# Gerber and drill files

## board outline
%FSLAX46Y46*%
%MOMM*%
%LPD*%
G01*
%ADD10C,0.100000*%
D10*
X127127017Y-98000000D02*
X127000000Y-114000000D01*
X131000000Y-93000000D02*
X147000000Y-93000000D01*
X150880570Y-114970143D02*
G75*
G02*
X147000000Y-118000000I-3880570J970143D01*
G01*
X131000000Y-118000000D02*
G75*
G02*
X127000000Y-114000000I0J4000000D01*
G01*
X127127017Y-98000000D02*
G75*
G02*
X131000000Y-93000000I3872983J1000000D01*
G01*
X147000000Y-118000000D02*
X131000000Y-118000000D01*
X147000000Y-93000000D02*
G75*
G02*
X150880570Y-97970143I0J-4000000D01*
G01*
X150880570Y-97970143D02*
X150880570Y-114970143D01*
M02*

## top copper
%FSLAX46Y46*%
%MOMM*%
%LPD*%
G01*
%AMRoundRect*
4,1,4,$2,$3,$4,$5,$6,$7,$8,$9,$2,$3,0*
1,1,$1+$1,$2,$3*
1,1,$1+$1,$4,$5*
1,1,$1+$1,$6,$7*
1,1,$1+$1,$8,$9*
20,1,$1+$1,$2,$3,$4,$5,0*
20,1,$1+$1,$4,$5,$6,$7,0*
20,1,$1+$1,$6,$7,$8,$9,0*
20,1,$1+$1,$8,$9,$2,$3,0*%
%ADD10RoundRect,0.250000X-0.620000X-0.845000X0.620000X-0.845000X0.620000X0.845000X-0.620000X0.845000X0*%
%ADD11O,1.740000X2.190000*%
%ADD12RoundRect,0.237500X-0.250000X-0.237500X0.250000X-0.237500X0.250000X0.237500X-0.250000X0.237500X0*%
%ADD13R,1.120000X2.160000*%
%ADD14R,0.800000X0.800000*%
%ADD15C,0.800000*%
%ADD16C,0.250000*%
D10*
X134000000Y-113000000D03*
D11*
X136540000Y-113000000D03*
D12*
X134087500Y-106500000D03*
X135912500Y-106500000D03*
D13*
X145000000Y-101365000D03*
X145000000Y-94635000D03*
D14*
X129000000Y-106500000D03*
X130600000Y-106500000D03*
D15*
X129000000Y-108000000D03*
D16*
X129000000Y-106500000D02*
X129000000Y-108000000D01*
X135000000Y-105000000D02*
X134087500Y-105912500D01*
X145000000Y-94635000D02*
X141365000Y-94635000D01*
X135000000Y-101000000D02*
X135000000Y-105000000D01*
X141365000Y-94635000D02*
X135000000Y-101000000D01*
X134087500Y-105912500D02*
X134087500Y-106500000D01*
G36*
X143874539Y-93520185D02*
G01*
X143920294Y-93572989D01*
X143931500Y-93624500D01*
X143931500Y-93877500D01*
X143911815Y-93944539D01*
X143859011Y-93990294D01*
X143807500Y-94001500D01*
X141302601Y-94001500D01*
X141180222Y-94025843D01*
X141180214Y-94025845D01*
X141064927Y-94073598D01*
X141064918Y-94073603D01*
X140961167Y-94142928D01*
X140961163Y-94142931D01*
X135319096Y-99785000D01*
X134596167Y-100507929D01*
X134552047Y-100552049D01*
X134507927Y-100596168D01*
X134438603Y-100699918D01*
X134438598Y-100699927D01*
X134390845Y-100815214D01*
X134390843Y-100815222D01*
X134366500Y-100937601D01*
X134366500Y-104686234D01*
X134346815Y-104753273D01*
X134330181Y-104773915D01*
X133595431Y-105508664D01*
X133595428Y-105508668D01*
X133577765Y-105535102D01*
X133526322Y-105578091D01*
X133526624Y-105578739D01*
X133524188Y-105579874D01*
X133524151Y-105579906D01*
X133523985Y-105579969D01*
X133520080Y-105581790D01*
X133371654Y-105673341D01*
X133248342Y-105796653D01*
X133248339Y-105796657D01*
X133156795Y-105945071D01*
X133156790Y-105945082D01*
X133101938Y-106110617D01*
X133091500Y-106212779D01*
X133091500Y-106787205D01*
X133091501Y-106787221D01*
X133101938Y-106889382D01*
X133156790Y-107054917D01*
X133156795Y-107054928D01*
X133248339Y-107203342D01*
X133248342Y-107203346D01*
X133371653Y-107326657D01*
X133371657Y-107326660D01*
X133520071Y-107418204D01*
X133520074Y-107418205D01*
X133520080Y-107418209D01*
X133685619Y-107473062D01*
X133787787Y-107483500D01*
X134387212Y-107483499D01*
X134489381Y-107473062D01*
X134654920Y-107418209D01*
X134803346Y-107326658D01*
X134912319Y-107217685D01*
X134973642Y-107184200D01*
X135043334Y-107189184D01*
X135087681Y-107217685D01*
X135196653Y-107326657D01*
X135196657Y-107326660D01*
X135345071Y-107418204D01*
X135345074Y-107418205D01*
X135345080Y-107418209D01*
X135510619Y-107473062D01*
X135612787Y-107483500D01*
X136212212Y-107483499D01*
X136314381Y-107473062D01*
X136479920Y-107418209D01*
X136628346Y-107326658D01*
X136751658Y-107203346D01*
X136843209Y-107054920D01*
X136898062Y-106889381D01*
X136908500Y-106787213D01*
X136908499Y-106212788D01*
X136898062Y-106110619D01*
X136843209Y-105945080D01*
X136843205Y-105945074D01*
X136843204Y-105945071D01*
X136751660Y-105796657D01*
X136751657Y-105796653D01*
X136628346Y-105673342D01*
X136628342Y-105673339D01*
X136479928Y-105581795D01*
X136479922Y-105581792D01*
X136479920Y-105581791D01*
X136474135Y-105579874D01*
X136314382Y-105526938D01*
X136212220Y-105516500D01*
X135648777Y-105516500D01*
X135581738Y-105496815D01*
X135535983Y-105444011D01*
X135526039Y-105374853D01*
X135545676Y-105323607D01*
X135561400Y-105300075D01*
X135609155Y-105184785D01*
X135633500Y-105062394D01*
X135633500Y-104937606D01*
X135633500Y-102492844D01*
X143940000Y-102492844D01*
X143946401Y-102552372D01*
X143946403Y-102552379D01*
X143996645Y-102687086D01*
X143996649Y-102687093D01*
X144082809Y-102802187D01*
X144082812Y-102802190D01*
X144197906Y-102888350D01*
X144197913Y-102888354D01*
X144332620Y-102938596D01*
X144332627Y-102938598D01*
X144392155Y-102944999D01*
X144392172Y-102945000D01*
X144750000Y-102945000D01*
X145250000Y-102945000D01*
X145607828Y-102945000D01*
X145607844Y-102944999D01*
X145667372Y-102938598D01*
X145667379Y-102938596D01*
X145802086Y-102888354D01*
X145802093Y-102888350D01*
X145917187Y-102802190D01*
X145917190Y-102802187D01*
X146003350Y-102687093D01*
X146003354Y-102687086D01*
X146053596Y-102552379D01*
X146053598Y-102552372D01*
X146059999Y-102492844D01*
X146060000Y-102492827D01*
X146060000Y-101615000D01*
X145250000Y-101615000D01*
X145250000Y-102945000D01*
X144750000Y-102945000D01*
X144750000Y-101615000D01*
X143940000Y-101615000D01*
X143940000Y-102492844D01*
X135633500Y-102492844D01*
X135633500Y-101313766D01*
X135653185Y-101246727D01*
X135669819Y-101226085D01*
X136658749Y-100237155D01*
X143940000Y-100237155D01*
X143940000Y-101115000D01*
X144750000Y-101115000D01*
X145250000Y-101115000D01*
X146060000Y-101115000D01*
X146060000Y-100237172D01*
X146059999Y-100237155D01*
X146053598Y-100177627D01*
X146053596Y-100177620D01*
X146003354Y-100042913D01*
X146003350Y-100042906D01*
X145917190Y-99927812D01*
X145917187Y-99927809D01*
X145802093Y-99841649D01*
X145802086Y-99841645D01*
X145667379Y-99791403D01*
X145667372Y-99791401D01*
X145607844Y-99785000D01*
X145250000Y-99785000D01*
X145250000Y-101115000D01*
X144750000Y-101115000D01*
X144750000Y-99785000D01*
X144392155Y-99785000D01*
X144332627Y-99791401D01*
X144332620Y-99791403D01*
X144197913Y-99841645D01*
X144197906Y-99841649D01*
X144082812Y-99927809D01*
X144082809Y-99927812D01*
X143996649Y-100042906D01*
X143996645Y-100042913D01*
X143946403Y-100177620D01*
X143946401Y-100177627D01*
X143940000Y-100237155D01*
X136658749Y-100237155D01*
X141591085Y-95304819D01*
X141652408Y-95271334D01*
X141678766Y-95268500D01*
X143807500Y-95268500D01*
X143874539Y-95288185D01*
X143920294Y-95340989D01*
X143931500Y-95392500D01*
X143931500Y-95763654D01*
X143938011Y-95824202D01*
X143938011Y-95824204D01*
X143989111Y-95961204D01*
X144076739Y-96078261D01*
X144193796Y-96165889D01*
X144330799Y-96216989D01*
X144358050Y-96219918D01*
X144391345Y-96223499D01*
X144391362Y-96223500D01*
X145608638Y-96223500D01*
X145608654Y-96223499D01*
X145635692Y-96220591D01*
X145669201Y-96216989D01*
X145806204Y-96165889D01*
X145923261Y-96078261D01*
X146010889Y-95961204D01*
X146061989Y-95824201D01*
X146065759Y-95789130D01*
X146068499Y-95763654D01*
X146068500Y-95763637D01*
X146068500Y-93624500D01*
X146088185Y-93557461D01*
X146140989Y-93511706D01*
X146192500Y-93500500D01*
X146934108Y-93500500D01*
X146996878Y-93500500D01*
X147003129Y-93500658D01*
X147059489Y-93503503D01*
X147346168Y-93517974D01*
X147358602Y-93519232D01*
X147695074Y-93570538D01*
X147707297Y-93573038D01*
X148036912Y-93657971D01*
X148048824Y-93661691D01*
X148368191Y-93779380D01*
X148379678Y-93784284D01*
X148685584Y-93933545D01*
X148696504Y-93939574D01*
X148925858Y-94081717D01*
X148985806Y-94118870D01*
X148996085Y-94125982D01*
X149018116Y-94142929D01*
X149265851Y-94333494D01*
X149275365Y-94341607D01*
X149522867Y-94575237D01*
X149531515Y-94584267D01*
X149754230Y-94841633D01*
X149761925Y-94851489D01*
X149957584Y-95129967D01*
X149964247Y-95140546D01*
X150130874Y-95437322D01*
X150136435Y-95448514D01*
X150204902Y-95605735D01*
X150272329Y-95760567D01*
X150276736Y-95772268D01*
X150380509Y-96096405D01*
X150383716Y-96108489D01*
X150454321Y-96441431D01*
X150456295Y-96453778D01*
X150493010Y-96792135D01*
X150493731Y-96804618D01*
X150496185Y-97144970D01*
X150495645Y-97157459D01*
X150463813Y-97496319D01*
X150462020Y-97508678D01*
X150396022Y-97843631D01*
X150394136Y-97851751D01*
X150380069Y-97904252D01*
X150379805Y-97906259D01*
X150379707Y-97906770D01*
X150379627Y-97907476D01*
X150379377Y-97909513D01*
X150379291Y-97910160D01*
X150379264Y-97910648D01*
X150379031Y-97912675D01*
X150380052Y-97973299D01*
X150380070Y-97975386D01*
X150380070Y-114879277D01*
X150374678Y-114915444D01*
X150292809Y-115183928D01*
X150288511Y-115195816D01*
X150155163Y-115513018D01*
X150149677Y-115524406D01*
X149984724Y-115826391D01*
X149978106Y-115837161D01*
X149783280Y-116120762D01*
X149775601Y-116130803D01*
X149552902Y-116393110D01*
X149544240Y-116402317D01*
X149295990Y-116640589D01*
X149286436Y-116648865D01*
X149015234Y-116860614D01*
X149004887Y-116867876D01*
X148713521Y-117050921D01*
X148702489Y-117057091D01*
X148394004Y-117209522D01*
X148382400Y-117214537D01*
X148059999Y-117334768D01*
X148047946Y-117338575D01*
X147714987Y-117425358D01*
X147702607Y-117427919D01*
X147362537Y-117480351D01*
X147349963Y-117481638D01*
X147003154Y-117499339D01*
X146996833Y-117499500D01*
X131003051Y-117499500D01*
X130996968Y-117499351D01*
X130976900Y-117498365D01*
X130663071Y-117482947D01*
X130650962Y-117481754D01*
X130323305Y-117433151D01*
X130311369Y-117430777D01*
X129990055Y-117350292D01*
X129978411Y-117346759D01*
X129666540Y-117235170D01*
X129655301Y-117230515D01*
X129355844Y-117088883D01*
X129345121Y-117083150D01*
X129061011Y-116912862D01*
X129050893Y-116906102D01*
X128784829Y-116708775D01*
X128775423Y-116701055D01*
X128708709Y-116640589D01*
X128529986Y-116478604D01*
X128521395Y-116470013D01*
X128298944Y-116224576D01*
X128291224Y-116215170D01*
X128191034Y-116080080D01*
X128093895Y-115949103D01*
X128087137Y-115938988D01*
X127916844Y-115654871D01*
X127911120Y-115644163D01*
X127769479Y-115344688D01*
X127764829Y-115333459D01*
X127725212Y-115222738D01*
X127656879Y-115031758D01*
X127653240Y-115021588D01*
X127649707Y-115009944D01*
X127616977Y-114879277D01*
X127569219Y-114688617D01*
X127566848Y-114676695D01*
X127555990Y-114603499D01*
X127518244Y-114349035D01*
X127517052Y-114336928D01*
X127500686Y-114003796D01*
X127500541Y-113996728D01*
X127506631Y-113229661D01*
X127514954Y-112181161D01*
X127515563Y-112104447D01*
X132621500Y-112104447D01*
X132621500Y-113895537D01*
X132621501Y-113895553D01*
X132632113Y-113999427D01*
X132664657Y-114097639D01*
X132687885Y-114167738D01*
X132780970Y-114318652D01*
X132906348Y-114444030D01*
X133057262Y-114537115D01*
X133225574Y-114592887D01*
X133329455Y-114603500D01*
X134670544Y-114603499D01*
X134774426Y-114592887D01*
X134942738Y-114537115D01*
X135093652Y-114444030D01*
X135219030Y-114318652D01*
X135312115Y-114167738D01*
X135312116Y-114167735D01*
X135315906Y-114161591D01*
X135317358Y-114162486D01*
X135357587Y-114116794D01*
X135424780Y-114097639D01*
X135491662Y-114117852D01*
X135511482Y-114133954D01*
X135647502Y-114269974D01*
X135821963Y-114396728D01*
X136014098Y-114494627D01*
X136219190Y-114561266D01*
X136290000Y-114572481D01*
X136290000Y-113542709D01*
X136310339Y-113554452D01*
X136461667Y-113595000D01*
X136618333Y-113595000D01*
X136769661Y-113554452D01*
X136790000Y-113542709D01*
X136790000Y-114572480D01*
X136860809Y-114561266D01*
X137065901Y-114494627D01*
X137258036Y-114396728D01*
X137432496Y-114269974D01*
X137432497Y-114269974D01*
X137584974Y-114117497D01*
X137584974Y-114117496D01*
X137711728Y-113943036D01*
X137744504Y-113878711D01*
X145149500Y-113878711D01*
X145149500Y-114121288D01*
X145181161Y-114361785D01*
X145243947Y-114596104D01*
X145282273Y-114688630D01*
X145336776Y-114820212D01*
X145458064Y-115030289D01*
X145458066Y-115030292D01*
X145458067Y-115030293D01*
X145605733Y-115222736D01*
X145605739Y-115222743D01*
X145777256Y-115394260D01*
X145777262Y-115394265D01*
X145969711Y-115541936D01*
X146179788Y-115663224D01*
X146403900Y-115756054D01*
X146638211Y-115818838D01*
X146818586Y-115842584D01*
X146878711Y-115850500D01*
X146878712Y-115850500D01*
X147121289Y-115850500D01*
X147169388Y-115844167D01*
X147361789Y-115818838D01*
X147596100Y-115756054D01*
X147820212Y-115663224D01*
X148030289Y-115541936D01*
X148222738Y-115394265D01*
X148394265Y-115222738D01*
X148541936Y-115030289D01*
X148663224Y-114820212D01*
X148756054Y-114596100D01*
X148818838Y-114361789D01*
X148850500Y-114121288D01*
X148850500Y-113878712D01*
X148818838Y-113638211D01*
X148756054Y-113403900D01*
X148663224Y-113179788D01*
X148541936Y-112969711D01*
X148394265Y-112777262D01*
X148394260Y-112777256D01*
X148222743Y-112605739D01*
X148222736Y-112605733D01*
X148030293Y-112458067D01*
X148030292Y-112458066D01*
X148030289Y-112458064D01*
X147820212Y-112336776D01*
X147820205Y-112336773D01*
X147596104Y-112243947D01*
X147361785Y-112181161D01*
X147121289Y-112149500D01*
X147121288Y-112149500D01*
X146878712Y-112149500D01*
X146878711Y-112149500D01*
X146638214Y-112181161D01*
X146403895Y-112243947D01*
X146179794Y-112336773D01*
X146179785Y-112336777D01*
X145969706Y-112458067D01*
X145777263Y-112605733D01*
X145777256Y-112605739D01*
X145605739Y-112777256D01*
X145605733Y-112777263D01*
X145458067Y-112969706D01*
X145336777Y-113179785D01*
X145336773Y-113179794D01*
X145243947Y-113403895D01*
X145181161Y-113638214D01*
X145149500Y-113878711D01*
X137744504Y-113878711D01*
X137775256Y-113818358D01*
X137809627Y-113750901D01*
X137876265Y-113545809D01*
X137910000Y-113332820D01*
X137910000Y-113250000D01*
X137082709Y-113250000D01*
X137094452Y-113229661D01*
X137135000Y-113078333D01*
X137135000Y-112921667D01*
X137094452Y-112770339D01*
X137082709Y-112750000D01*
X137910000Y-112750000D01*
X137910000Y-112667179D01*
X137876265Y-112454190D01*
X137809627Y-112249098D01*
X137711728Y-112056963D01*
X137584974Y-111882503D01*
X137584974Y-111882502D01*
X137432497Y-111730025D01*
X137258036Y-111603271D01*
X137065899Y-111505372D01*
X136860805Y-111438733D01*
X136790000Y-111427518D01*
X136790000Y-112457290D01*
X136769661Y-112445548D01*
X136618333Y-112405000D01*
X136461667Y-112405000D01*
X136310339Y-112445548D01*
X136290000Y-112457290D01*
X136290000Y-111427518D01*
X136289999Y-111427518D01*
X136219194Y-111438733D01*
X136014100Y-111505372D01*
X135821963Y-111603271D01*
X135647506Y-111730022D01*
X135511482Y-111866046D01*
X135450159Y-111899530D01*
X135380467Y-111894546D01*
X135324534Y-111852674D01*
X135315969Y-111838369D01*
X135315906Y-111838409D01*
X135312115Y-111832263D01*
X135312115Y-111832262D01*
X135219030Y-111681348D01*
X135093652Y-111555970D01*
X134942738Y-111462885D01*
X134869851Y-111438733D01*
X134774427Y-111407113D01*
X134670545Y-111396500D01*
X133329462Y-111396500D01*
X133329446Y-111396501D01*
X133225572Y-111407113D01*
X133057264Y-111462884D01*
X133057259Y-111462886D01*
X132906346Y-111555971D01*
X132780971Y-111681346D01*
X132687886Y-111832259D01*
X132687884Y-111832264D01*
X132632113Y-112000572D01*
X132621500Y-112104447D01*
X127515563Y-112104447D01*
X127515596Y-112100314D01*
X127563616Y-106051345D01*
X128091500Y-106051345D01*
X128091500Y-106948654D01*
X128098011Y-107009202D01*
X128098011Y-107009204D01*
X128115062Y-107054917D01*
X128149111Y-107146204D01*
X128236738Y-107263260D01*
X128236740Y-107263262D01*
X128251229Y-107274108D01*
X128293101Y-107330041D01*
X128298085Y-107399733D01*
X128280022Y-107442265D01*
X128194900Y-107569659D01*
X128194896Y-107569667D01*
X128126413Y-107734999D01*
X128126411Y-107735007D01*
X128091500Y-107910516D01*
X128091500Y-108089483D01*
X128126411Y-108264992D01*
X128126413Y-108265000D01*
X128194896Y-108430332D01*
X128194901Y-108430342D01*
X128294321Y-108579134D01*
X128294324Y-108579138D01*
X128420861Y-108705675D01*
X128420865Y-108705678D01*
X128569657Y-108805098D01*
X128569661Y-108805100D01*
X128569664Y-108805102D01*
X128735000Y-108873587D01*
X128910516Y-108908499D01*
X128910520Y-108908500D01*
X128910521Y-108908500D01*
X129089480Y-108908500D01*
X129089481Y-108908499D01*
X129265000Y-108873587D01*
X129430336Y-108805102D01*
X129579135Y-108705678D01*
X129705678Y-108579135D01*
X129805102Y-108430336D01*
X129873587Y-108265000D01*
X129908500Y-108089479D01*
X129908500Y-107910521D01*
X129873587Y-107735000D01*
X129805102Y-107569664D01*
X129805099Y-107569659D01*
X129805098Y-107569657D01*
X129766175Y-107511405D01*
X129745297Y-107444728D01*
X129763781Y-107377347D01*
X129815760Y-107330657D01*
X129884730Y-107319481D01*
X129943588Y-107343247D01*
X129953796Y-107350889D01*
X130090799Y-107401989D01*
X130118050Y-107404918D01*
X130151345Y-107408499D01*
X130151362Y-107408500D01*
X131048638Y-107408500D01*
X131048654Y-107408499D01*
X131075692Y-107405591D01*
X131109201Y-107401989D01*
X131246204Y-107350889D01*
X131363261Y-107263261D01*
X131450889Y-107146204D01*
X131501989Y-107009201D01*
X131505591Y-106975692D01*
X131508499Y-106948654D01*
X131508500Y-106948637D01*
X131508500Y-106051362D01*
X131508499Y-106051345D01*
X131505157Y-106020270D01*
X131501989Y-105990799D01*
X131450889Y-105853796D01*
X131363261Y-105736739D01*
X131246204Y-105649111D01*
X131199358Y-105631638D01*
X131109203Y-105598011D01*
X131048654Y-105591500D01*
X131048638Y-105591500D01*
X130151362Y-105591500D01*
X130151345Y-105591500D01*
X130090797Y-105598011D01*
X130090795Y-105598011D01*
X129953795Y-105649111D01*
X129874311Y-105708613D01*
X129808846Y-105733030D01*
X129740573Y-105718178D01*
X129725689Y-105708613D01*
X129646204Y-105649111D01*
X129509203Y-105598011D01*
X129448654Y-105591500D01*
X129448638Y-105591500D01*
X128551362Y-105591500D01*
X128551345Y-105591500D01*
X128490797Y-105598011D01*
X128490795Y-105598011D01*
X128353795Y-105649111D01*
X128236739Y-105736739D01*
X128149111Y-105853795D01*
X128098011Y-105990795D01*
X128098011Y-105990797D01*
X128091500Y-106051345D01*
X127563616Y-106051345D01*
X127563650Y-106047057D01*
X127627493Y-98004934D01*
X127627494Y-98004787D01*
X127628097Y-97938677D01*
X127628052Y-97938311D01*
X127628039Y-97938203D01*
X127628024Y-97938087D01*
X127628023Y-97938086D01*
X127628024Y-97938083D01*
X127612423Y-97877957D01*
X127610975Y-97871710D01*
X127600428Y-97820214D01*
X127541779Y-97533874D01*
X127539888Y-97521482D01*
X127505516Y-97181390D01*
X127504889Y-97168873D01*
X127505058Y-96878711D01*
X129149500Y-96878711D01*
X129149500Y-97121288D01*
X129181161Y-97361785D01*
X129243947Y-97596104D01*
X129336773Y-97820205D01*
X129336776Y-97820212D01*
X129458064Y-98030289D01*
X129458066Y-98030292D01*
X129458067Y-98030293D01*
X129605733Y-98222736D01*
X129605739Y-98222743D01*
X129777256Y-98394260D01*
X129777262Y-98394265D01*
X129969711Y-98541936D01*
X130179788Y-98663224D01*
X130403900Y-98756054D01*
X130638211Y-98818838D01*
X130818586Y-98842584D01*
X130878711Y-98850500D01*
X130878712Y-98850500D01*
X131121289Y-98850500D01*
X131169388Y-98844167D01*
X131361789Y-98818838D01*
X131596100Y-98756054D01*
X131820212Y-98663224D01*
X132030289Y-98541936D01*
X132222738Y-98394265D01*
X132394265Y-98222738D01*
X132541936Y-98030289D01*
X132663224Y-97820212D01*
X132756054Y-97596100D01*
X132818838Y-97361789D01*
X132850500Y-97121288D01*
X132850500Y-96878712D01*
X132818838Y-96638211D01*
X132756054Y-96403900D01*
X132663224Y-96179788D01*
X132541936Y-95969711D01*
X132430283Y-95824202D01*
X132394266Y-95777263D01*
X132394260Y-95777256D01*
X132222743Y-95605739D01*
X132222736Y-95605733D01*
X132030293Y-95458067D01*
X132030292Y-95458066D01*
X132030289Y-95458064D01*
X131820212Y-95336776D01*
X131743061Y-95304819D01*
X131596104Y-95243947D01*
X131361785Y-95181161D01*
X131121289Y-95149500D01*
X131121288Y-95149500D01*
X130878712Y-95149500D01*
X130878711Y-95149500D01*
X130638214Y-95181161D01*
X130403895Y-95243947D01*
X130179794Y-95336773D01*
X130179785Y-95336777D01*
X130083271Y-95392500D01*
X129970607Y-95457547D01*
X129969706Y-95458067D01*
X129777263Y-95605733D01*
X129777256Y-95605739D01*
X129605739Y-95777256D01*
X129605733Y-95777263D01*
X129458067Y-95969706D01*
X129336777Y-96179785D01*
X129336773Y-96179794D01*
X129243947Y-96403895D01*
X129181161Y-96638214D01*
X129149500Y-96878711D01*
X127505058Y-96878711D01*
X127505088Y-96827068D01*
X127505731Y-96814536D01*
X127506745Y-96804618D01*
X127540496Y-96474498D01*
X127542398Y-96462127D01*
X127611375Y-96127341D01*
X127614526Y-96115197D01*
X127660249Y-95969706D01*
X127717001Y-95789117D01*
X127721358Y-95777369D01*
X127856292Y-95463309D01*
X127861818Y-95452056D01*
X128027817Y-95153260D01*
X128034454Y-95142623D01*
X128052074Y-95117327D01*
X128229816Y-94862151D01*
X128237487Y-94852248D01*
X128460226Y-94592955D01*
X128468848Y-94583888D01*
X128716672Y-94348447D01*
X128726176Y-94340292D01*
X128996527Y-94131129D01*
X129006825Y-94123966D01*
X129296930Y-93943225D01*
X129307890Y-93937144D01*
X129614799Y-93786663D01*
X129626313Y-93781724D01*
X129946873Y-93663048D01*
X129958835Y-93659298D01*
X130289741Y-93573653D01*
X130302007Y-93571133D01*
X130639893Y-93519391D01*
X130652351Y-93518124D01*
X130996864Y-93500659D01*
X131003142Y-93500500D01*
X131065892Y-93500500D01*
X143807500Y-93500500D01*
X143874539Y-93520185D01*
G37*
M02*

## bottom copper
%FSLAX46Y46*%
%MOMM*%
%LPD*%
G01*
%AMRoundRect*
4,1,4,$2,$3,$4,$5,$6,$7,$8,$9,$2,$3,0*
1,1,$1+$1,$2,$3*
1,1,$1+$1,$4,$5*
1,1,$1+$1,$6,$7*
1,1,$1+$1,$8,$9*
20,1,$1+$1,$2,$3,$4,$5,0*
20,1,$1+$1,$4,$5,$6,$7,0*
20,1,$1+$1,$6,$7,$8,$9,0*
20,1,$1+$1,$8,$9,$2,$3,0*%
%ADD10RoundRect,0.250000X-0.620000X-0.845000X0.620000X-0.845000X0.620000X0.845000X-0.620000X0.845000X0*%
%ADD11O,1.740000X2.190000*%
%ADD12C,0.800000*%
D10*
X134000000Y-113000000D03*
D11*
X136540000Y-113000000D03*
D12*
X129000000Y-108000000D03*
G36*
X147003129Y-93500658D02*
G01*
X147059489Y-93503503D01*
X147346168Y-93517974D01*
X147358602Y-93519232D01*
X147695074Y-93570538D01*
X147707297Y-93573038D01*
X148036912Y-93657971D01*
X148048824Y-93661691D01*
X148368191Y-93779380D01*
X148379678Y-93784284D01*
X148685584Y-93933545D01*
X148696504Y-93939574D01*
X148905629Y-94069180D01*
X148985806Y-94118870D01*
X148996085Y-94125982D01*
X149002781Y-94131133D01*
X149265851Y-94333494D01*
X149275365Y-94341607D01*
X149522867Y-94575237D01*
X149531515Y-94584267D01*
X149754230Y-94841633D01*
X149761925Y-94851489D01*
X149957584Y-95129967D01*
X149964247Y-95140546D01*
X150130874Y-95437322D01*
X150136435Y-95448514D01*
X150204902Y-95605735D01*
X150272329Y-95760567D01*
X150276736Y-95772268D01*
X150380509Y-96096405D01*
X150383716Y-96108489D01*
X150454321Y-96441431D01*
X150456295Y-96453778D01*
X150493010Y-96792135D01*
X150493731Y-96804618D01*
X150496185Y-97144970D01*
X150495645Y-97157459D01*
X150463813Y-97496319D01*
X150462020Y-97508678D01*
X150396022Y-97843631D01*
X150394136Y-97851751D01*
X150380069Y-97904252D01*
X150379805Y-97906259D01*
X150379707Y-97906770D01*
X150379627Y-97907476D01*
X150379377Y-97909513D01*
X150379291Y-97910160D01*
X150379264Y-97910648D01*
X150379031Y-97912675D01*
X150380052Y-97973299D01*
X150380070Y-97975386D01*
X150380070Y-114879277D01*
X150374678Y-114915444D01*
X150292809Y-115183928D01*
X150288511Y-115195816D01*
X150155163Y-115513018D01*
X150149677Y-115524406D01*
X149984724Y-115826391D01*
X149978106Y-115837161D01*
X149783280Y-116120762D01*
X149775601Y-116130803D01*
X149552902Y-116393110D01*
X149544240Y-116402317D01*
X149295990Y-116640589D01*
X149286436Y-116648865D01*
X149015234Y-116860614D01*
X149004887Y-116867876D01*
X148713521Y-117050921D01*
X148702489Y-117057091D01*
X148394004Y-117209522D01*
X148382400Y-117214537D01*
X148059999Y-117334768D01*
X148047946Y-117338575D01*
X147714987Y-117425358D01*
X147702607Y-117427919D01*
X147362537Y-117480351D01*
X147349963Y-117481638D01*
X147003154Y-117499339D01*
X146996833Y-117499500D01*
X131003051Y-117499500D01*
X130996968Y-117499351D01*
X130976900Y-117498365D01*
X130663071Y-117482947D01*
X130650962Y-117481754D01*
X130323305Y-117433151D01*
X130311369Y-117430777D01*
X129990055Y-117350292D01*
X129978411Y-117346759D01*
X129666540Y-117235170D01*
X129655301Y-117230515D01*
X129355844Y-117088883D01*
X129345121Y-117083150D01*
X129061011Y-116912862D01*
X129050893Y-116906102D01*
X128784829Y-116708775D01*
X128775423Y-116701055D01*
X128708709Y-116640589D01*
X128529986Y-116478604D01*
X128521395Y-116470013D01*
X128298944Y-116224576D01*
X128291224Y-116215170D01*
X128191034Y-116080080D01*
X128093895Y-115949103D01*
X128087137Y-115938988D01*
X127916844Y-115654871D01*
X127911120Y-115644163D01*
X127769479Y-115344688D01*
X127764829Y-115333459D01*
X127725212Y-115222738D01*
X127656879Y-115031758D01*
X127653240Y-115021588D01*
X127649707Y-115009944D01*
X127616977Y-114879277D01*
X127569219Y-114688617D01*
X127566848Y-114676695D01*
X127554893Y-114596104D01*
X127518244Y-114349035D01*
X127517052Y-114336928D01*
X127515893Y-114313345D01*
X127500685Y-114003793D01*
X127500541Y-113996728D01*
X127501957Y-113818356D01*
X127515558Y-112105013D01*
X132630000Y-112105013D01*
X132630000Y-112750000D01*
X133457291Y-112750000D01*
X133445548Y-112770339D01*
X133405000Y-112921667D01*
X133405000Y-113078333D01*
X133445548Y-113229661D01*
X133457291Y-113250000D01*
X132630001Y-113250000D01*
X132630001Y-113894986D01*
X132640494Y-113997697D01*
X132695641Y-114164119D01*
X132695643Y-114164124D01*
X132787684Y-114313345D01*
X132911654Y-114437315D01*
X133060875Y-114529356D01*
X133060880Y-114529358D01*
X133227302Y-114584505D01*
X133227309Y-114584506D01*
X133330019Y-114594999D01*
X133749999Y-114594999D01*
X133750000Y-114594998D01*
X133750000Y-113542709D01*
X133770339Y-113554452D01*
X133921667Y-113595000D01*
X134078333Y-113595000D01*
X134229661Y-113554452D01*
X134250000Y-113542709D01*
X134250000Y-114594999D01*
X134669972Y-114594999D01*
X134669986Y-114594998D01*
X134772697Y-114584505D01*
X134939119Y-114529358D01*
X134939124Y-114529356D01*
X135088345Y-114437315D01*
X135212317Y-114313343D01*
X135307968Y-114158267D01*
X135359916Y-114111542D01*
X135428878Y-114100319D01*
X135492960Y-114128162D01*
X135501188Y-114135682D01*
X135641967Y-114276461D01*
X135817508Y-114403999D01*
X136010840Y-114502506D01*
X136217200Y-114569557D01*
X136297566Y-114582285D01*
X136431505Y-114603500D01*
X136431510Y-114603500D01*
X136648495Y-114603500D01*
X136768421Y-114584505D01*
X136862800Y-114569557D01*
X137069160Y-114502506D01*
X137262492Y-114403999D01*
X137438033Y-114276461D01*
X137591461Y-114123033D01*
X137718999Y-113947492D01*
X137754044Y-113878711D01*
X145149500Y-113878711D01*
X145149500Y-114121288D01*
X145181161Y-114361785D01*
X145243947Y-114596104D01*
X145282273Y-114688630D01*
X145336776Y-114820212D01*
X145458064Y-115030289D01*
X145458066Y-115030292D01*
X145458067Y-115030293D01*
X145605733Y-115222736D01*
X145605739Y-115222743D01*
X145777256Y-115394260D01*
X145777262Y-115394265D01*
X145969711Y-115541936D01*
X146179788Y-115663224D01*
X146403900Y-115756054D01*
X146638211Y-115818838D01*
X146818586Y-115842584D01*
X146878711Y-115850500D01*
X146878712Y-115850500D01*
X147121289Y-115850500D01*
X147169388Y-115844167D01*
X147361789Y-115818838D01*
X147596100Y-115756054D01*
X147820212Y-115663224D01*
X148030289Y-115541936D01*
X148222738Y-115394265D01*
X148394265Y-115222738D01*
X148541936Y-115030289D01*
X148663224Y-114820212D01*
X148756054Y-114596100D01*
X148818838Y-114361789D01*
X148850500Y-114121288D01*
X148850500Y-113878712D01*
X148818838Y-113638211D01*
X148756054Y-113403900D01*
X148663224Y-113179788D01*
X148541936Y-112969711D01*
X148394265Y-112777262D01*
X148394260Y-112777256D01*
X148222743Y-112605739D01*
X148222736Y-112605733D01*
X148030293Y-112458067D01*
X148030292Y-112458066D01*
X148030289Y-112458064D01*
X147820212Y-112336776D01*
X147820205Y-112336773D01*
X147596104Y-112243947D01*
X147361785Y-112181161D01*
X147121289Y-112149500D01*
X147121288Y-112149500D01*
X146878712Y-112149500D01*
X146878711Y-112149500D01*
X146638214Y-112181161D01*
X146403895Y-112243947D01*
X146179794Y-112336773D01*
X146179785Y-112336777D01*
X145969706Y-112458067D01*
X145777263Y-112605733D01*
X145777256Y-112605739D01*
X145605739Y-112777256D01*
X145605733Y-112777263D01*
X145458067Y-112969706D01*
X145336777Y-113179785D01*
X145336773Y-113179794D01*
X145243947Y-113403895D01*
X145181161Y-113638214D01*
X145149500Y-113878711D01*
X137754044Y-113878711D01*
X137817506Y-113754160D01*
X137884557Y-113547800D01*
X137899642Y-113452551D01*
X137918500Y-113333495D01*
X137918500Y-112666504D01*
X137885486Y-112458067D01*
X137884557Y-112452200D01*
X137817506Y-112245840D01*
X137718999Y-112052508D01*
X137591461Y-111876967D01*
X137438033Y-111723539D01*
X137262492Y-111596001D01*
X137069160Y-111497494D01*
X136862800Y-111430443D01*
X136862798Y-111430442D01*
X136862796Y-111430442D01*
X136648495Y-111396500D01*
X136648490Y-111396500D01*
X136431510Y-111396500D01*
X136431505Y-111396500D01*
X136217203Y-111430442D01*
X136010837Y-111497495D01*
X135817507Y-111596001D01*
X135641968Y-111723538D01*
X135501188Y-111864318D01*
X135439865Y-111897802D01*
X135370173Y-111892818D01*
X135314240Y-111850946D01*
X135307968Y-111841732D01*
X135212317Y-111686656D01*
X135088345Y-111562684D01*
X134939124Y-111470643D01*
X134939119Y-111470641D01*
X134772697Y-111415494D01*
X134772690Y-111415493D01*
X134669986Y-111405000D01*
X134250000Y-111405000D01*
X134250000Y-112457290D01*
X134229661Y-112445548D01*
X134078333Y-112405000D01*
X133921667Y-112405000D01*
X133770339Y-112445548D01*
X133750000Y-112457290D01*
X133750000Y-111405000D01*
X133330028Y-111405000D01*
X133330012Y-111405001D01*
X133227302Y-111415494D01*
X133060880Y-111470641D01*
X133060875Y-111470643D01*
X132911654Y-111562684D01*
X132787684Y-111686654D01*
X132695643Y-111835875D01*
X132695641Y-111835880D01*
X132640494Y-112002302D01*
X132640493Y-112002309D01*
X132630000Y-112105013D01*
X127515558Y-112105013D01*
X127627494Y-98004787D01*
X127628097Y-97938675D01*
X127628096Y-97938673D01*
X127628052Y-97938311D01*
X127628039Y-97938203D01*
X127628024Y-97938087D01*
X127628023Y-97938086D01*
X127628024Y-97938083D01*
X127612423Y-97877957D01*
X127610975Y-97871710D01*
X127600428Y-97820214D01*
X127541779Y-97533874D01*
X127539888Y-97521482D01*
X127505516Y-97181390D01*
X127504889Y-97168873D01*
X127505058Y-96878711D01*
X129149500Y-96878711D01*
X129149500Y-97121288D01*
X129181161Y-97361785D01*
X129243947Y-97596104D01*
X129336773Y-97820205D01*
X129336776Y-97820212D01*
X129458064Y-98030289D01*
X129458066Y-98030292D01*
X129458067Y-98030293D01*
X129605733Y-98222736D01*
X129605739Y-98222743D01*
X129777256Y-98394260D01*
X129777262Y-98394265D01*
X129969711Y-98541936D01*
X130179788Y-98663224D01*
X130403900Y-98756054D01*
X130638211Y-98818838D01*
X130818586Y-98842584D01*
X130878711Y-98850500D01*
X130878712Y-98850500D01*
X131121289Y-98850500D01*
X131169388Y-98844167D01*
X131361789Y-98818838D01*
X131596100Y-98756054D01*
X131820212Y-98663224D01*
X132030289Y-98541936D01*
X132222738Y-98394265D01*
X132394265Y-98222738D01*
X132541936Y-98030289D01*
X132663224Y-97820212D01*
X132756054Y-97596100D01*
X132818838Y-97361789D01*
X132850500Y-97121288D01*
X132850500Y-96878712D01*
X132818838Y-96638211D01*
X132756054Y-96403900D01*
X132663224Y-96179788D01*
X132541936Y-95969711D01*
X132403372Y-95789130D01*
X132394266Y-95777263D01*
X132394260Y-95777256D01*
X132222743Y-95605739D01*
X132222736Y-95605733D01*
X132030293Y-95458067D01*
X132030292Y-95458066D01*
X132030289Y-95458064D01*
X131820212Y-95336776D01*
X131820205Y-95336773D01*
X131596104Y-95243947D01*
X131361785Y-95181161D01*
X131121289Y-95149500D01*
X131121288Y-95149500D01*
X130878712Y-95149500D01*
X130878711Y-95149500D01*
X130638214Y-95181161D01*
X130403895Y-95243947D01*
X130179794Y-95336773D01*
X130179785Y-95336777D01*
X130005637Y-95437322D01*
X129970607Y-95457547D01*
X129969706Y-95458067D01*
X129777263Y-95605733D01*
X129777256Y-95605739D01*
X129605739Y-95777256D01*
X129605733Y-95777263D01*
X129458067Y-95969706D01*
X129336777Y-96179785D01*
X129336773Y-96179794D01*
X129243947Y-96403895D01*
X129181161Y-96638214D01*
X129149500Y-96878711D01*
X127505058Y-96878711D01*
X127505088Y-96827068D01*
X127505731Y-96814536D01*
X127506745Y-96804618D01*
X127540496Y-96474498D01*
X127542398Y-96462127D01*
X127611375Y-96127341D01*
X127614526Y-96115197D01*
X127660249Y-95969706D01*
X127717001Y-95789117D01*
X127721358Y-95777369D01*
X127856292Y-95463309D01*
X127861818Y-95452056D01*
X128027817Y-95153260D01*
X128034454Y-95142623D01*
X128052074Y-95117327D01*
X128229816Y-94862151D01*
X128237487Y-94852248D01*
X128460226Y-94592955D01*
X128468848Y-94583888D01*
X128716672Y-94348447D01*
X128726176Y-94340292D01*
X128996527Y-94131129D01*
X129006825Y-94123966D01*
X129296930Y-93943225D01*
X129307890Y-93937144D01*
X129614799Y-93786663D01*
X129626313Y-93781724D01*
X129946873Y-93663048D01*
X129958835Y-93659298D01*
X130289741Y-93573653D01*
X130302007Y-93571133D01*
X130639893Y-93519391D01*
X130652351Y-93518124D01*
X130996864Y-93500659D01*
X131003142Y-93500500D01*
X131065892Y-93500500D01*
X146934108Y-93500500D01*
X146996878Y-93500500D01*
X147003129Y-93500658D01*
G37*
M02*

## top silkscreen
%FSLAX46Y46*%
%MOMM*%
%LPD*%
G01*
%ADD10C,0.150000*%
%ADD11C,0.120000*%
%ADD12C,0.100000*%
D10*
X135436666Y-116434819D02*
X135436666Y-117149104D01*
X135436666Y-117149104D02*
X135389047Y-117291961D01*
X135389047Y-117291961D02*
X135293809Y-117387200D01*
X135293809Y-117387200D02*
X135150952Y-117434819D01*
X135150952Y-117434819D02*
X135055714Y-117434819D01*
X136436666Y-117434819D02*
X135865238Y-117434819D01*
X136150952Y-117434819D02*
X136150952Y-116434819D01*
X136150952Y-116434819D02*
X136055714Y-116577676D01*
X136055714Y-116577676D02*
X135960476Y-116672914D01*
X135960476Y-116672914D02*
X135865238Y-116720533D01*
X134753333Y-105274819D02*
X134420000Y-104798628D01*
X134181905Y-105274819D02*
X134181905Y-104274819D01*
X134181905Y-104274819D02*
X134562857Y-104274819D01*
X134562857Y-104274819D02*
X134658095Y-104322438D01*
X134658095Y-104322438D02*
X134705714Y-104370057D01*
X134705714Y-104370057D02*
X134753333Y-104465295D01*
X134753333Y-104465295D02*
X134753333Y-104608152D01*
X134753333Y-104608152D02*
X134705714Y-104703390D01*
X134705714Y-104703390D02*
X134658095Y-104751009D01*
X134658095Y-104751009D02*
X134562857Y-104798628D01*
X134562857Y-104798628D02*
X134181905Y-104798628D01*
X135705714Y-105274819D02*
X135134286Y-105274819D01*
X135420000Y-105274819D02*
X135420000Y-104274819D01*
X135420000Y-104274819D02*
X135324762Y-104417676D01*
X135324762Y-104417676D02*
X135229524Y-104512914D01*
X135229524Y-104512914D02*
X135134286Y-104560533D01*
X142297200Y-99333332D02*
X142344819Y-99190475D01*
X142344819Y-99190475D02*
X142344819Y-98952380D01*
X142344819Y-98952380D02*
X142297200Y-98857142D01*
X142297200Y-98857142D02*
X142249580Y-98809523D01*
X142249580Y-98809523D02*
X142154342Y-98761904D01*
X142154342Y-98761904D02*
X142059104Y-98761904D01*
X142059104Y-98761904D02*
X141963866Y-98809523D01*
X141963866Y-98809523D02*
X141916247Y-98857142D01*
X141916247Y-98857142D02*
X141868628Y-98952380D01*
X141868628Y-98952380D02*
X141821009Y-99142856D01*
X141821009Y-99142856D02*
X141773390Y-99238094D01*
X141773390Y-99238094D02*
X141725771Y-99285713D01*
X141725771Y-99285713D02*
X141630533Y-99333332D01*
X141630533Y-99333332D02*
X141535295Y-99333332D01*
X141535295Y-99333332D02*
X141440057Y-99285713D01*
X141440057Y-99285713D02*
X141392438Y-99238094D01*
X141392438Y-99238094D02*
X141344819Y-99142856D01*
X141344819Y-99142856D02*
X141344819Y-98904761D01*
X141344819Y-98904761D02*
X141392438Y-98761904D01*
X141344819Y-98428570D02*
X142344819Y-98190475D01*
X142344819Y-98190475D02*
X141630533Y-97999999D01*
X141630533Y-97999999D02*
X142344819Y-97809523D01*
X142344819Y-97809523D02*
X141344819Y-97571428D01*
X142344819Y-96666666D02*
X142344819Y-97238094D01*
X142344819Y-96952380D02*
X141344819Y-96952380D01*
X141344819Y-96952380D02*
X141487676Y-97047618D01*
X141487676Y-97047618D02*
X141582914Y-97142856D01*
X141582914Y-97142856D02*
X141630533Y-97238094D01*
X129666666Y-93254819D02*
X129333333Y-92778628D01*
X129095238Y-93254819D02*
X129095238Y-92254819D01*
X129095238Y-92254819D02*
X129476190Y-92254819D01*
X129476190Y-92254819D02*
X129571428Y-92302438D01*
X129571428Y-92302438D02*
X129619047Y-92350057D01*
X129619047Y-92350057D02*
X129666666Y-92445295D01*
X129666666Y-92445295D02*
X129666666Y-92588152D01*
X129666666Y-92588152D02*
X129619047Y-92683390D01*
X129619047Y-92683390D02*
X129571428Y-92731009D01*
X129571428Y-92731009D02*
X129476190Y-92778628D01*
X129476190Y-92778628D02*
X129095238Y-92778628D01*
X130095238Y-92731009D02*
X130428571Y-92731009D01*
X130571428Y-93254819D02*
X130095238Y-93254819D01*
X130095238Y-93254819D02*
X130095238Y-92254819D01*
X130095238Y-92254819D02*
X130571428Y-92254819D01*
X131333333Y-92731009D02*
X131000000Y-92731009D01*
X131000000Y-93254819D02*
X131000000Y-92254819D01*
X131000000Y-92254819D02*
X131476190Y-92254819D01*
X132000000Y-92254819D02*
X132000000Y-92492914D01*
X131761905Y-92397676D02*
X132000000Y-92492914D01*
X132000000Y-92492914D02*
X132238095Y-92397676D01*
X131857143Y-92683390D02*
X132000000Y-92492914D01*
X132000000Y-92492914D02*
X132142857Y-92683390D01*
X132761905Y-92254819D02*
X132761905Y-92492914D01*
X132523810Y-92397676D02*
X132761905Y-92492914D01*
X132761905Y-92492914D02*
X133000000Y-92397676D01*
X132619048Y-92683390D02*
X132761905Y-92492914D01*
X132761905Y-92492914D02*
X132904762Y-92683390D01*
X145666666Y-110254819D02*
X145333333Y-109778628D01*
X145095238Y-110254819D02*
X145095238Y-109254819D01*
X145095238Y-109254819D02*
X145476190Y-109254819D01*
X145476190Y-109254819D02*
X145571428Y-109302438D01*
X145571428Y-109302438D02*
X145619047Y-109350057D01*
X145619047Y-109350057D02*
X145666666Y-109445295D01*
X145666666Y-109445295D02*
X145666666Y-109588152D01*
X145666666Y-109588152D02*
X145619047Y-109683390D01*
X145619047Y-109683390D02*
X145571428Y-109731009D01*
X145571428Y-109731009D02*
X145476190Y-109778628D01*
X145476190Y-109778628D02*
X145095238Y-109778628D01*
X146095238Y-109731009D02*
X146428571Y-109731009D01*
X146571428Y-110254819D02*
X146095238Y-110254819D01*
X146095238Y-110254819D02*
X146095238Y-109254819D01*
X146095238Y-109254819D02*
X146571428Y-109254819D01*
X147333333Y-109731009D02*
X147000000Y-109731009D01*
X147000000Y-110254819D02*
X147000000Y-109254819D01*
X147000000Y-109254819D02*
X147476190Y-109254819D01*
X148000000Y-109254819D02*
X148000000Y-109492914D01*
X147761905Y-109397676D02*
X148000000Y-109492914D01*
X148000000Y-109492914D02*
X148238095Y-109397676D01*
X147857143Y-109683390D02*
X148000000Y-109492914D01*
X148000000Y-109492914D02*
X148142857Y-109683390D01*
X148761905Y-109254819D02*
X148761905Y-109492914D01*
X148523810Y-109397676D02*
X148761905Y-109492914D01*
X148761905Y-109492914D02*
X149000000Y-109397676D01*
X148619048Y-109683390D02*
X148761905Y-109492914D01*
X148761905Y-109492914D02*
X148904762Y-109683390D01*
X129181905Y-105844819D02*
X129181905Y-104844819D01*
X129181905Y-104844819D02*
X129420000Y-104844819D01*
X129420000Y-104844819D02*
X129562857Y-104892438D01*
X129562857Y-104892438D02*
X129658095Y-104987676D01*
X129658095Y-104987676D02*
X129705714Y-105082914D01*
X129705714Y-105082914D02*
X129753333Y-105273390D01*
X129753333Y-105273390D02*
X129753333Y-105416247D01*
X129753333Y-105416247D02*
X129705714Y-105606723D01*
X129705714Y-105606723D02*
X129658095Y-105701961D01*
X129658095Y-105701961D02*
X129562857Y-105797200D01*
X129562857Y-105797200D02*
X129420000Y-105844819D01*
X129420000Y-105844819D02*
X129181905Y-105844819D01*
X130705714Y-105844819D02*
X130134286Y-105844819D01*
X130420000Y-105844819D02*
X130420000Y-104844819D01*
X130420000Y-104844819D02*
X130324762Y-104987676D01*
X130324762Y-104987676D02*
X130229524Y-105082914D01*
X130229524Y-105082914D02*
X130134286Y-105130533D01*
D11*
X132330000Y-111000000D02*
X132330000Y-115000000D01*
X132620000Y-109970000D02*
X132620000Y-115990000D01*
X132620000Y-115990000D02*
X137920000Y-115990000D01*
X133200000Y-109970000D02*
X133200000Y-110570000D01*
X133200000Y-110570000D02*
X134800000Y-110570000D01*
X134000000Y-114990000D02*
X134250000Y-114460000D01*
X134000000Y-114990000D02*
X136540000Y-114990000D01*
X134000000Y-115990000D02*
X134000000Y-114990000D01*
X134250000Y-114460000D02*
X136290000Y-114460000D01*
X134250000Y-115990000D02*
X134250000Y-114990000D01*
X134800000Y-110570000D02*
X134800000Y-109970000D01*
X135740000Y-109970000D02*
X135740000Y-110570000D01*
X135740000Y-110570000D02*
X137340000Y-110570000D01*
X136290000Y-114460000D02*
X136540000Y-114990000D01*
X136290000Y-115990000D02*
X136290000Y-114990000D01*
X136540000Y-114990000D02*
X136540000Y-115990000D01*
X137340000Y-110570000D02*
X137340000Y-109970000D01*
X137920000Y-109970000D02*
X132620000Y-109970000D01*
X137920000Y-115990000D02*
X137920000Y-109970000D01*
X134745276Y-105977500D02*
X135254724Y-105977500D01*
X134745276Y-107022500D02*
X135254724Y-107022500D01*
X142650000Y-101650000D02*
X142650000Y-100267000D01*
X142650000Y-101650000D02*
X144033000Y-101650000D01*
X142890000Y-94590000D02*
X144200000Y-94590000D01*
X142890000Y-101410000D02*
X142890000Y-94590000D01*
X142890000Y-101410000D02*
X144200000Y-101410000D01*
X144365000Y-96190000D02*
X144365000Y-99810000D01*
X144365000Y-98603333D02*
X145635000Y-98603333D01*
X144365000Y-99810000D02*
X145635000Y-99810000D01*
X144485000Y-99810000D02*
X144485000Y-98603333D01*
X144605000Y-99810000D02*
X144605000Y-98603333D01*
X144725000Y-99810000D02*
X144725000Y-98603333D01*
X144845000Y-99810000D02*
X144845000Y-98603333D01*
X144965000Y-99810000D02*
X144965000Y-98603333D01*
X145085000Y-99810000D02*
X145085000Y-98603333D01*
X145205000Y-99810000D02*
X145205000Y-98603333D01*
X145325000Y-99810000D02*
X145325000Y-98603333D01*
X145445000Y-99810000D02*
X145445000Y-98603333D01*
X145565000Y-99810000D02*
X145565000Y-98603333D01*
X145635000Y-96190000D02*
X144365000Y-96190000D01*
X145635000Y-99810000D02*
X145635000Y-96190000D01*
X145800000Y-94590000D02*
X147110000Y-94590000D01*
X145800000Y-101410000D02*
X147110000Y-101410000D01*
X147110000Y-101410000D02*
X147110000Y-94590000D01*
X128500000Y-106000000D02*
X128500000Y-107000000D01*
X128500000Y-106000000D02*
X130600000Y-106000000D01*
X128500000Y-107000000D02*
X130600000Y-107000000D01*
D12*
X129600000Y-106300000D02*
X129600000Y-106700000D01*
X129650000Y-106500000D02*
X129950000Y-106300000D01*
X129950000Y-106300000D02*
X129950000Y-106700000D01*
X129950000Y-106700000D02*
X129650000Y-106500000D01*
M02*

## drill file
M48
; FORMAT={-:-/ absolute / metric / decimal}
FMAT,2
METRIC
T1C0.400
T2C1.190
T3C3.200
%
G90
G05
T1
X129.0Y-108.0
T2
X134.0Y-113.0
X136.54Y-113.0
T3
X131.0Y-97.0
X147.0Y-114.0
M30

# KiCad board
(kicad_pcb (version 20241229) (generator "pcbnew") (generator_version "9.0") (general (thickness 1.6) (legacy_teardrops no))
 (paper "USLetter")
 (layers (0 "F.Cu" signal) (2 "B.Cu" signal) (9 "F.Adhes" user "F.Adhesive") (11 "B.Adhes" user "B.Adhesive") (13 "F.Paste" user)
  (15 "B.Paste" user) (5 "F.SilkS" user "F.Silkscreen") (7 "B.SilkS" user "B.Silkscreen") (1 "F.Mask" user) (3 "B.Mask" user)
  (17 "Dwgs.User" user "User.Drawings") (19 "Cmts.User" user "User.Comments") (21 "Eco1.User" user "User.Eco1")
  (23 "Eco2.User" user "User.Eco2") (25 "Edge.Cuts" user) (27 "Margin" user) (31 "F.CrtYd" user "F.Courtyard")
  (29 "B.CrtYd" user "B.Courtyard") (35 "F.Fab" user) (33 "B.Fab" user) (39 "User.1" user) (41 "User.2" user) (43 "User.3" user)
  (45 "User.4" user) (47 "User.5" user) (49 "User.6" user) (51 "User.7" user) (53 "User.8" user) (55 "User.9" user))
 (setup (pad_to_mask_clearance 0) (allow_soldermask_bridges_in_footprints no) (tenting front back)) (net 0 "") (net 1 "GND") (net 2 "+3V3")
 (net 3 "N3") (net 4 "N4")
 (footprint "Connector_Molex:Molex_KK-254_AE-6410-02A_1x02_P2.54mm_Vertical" (layer "F.Cu") (at 134 113)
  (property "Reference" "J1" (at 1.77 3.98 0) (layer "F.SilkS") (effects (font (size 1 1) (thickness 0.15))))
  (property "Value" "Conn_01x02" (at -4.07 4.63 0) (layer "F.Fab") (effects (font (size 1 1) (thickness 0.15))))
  (fp_line (start -1.67 -2) (end -1.67 2) (stroke (width 0.12) (type solid)) (layer "F.SilkS"))
  (fp_line (start -1.38 -3.03) (end -1.38 2.99) (stroke (width 0.12) (type solid)) (layer "F.SilkS"))
  (fp_line (start -1.38 2.99) (end 3.92 2.99) (stroke (width 0.12) (type solid)) (layer "F.SilkS"))
  (fp_line (start -0.8 -3.03) (end -0.8 -2.43) (stroke (width 0.12) (type solid)) (layer "F.SilkS"))
  (fp_line (start -0.8 -2.43) (end 0.8 -2.43) (stroke (width 0.12) (type solid)) (layer "F.SilkS"))
  (fp_line (start 0 1.99) (end 0.25 1.46) (stroke (width 0.12) (type solid)) (layer "F.SilkS"))
  (fp_line (start 0 1.99) (end 2.54 1.99) (stroke (width 0.12) (type solid)) (layer "F.SilkS"))
  (fp_line (start 0 2.99) (end 0 1.99) (stroke (width 0.12) (type solid)) (layer "F.SilkS"))
  (fp_line (start 0.25 1.46) (end 2.29 1.46) (stroke (width 0.12) (type solid)) (layer "F.SilkS"))
  (fp_line (start 0.25 2.99) (end 0.25 1.99) (stroke (width 0.12) (type solid)) (layer "F.SilkS"))
  (fp_line (start 0.8 -2.43) (end 0.8 -3.03) (stroke (width 0.12) (type solid)) (layer "F.SilkS"))
  (fp_line (start 1.74 -3.03) (end 1.74 -2.43) (stroke (width 0.12) (type solid)) (layer "F.SilkS"))
  (fp_line (start 1.74 -2.43) (end 3.34 -2.43) (stroke (width 0.12) (type solid)) (layer "F.SilkS"))
  (fp_line (start 2.29 1.46) (end 2.54 1.99) (stroke (width 0.12) (type solid)) (layer "F.SilkS"))
  (fp_line (start 2.29 2.99) (end 2.29 1.99) (stroke (width 0.12) (type solid)) (layer "F.SilkS"))
  (fp_line (start 2.54 1.99) (end 2.54 2.99) (stroke (width 0.12) (type solid)) (layer "F.SilkS"))
  (fp_line (start 3.34 -2.43) (end 3.34 -3.03) (stroke (width 0.12) (type solid)) (layer "F.SilkS"))
  (fp_line (start 3.92 -3.03) (end -1.38 -3.03) (stroke (width 0.12) (type solid)) (layer "F.SilkS"))
  (fp_line (start 3.92 2.99) (end 3.92 -3.03) (stroke (width 0.12) (type solid)) (layer "F.SilkS"))
  (pad "1" thru_hole roundrect (at 0 0) (size 1.74 2.19) (drill 1.19) (layers "*.Cu" "*.Mask") (remove_unused_layers no)
   (roundrect_rratio 0.143678) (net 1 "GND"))
  (pad "2" thru_hole oval (at 2.54 0) (size 1.74 2.19) (drill 1.19) (layers "*.Cu" "*.Mask") (remove_unused_layers no) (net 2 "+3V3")))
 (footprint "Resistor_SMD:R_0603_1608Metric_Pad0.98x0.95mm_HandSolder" (layer "F.Cu") (at 135 106.5)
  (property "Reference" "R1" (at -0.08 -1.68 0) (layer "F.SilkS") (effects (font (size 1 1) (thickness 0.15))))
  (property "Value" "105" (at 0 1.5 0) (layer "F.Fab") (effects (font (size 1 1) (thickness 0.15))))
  (fp_line (start -0.254724 -0.5225) (end 0.254724 -0.5225) (stroke (width 0.12) (type solid)) (layer "F.SilkS"))
  (fp_line (start -0.254724 0.5225) (end 0.254724 0.5225) (stroke (width 0.12) (type solid)) (layer "F.SilkS"))
  (pad "1" smd roundrect (at -0.9125 0) (size 0.975 0.95) (layers "F.Cu" "F.Mask" "F.Paste") (roundrect_rratio 0.25) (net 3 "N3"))
  (pad "2" smd roundrect (at 0.9125 0) (size 0.975 0.95) (layers "F.Cu" "F.Mask" "F.Paste") (roundrect_rratio 0.25) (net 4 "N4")))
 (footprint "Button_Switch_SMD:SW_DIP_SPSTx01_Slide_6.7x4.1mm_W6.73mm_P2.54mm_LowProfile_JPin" (layer "F.Cu") (at 145 98 90)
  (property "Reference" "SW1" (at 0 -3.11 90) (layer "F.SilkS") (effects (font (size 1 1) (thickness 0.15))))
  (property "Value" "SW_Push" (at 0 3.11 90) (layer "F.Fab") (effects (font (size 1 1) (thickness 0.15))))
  (fp_line (start -3.65 -2.35) (end -2.267 -2.35) (stroke (width 0.12) (type solid)) (layer "F.SilkS"))
  (fp_line (start -3.65 -2.35) (end -3.65 -0.967) (stroke (width 0.12) (type solid)) (layer "F.SilkS"))
  (fp_line (start 3.41 -2.11) (end 3.41 -0.8) (stroke (width 0.12) (type solid)) (layer "F.SilkS"))
  (fp_line (start -3.41 -2.11) (end 3.41 -2.11) (stroke (width 0.12) (type solid)) (layer "F.SilkS"))
  (fp_line (start -3.41 -2.11) (end -3.41 -0.8) (stroke (width 0.12) (type solid)) (layer "F.SilkS"))
  (fp_line (start 1.81 -0.635) (end -1.81 -0.635) (stroke (width 0.12) (type solid)) (layer "F.SilkS"))
  (fp_line (start -0.603333 -0.635) (end -0.603333 0.635) (stroke (width 0.12) (type solid)) (layer "F.SilkS"))
  (fp_line (start -1.81 -0.635) (end -1.81 0.635) (stroke (width 0.12) (type solid)) (layer "F.SilkS"))
  (fp_line (start -1.81 -0.515) (end -0.603333 -0.515) (stroke (width 0.12) (type solid)) (layer "F.SilkS"))
  (fp_line (start -1.81 -0.395) (end -0.603333 -0.395) (stroke (width 0.12) (type solid)) (layer "F.SilkS"))
  (fp_line (start -1.81 -0.275) (end -0.603333 -0.275) (stroke (width 0.12) (type solid)) (layer "F.SilkS"))
  (fp_line (start -1.81 -0.155) (end -0.603333 -0.155) (stroke (width 0.12) (type solid)) (layer "F.SilkS"))
  (fp_line (start -1.81 -0.035) (end -0.603333 -0.035) (stroke (width 0.12) (type solid)) (layer "F.SilkS"))
  (fp_line (start -1.81 0.085) (end -0.603333 0.085) (stroke (width 0.12) (type solid)) (layer "F.SilkS"))
  (fp_line (start -1.81 0.205) (end -0.603333 0.205) (stroke (width 0.12) (type solid)) (layer "F.SilkS"))
  (fp_line (start -1.81 0.325) (end -0.603333 0.325) (stroke (width 0.12) (type solid)) (layer "F.SilkS"))
  (fp_line (start -1.81 0.445) (end -0.603333 0.445) (stroke (width 0.12) (type solid)) (layer "F.SilkS"))
  (fp_line (start -1.81 0.565) (end -0.603333 0.565) (stroke (width 0.12) (type solid)) (layer "F.SilkS"))
  (fp_line (start 1.81 0.635) (end 1.81 -0.635) (stroke (width 0.12) (type solid)) (layer "F.SilkS"))
  (fp_line (start -1.81 0.635) (end 1.81 0.635) (stroke (width 0.12) (type solid)) (layer "F.SilkS"))
  (fp_line (start 3.41 0.8) (end 3.41 2.11) (stroke (width 0.12) (type solid)) (layer "F.SilkS"))
  (fp_line (start -3.41 0.8) (end -3.41 2.11) (stroke (width 0.12) (type solid)) (layer "F.SilkS"))
  (fp_line (start -3.41 2.11) (end 3.41 2.11) (stroke (width 0.12) (type solid)) (layer "F.SilkS"))
  (pad "1" smd rect (at -3.365 0 90) (size 2.16 1.12) (layers "F.Cu" "F.Mask" "F.Paste") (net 2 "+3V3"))
  (pad "2" smd rect (at 3.365 0 90) (size 2.16 1.12) (layers "F.Cu" "F.Mask" "F.Paste") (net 3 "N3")))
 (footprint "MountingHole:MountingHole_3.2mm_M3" (layer "F.Cu") (at 131 97)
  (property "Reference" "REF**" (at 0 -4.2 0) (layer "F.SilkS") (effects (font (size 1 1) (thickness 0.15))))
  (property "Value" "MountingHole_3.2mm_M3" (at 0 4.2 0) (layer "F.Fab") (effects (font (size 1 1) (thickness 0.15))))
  (pad "" np_thru_hole circle (at 0 0) (size 3.2 3.2) (drill 3.2) (layers "*.Cu" "*.Mask")))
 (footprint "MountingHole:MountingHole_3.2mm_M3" (layer "F.Cu") (at 147 114)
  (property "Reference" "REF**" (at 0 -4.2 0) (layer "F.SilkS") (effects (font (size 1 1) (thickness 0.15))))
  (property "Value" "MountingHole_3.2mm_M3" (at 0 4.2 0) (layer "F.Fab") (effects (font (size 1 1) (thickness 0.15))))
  (pad "" np_thru_hole circle (at 0 0) (size 3.2 3.2) (drill 3.2) (layers "*.Cu" "*.Mask")))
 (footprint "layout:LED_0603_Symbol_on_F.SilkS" (layer "F.Cu") (at 129.8 106.5)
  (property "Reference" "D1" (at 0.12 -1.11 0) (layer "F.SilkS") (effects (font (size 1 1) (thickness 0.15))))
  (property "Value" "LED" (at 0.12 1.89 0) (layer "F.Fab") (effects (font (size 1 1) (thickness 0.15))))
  (fp_line (start -1.3 -0.5) (end -1.3 0.5) (stroke (width 0.12) (type solid)) (layer "F.SilkS"))
  (fp_line (start -1.3 -0.5) (end 0.8 -0.5) (stroke (width 0.12) (type solid)) (layer "F.SilkS"))
  (fp_line (start -1.3 0.5) (end 0.8 0.5) (stroke (width 0.12) (type solid)) (layer "F.SilkS"))
  (fp_line (start -0.2 -0.2) (end -0.2 0.2) (stroke (width 0.1) (type solid)) (layer "F.SilkS"))
  (fp_line (start -0.15 0) (end 0.15 -0.2) (stroke (width 0.1) (type solid)) (layer "F.SilkS"))
  (fp_line (start 0.15 -0.2) (end 0.15 0.2) (stroke (width 0.1) (type solid)) (layer "F.SilkS"))
  (fp_line (start 0.15 0.2) (end -0.15 0) (stroke (width 0.1) (type solid)) (layer "F.SilkS"))
  (pad "1" smd rect (at -0.8 0 180) (size 0.8 0.8) (layers "F.Cu" "F.Mask" "F.Paste") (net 1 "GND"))
  (pad "2" smd rect (at 0.8 0 180) (size 0.8 0.8) (layers "F.Cu" "F.Mask" "F.Paste") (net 4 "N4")))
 (gr_line (start 127.127017 98) (end 127 114) (stroke (width 0.1) (type default)) (layer "Edge.Cuts"))
 (gr_line (start 131 93) (end 147 93) (stroke (width 0.1) (type default)) (layer "Edge.Cuts"))
 (gr_arc (start 150.88057 114.970143) (mid 149.461649 117.152822) (end 147 118) (stroke (width 0.1) (type default)) (layer "Edge.Cuts"))
 (gr_arc (start 131 118) (mid 128.171573 116.828427) (end 127 114) (stroke (width 0.1) (type default)) (layer "Edge.Cuts"))
 (gr_arc (start 127.127017 98) (mid 127.837723 94.55051) (end 131 93) (stroke (width 0.1) (type default)) (layer "Edge.Cuts"))
 (gr_line (start 147 118) (end 131 118) (stroke (width 0.1) (type default)) (layer "Edge.Cuts"))
 (gr_arc (start 147 93) (mid 150.152822 94.538351) (end 150.88057 97.970143) (stroke (width 0.1) (type default)) (layer "Edge.Cuts"))
 (gr_line (start 150.88057 97.970143) (end 150.88057 114.970143) (stroke (width 0.1) (type default)) (layer "Edge.Cuts"))
 (segment (start 129 106.5) (end 129 108) (width 0.25) (layer "F.Cu") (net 1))
 (via (at 129 108) (size 0.8) (drill 0.4) (layers "F.Cu" "B.Cu") (free yes) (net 1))
 (segment (start 135 105) (end 134.0875 105.9125) (width 0.25) (layer "F.Cu") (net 3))
 (segment (start 145 94.635) (end 141.365 94.635) (width 0.25) (layer "F.Cu") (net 3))
 (segment (start 135 101) (end 135 105) (width 0.25) (layer "F.Cu") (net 3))
 (segment (start 141.365 94.635) (end 135 101) (width 0.25) (layer "F.Cu") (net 3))
 (segment (start 134.0875 105.9125) (end 134.0875 106.5) (width 0.25) (layer "F.Cu") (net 3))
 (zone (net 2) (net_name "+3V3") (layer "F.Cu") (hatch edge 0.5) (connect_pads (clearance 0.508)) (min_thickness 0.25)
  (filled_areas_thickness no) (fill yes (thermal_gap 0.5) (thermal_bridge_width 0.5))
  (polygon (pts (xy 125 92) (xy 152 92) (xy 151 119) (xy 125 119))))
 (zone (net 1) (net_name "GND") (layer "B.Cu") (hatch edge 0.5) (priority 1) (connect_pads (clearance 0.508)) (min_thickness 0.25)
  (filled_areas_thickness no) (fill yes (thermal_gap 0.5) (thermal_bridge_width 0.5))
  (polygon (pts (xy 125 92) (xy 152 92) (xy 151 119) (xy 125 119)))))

